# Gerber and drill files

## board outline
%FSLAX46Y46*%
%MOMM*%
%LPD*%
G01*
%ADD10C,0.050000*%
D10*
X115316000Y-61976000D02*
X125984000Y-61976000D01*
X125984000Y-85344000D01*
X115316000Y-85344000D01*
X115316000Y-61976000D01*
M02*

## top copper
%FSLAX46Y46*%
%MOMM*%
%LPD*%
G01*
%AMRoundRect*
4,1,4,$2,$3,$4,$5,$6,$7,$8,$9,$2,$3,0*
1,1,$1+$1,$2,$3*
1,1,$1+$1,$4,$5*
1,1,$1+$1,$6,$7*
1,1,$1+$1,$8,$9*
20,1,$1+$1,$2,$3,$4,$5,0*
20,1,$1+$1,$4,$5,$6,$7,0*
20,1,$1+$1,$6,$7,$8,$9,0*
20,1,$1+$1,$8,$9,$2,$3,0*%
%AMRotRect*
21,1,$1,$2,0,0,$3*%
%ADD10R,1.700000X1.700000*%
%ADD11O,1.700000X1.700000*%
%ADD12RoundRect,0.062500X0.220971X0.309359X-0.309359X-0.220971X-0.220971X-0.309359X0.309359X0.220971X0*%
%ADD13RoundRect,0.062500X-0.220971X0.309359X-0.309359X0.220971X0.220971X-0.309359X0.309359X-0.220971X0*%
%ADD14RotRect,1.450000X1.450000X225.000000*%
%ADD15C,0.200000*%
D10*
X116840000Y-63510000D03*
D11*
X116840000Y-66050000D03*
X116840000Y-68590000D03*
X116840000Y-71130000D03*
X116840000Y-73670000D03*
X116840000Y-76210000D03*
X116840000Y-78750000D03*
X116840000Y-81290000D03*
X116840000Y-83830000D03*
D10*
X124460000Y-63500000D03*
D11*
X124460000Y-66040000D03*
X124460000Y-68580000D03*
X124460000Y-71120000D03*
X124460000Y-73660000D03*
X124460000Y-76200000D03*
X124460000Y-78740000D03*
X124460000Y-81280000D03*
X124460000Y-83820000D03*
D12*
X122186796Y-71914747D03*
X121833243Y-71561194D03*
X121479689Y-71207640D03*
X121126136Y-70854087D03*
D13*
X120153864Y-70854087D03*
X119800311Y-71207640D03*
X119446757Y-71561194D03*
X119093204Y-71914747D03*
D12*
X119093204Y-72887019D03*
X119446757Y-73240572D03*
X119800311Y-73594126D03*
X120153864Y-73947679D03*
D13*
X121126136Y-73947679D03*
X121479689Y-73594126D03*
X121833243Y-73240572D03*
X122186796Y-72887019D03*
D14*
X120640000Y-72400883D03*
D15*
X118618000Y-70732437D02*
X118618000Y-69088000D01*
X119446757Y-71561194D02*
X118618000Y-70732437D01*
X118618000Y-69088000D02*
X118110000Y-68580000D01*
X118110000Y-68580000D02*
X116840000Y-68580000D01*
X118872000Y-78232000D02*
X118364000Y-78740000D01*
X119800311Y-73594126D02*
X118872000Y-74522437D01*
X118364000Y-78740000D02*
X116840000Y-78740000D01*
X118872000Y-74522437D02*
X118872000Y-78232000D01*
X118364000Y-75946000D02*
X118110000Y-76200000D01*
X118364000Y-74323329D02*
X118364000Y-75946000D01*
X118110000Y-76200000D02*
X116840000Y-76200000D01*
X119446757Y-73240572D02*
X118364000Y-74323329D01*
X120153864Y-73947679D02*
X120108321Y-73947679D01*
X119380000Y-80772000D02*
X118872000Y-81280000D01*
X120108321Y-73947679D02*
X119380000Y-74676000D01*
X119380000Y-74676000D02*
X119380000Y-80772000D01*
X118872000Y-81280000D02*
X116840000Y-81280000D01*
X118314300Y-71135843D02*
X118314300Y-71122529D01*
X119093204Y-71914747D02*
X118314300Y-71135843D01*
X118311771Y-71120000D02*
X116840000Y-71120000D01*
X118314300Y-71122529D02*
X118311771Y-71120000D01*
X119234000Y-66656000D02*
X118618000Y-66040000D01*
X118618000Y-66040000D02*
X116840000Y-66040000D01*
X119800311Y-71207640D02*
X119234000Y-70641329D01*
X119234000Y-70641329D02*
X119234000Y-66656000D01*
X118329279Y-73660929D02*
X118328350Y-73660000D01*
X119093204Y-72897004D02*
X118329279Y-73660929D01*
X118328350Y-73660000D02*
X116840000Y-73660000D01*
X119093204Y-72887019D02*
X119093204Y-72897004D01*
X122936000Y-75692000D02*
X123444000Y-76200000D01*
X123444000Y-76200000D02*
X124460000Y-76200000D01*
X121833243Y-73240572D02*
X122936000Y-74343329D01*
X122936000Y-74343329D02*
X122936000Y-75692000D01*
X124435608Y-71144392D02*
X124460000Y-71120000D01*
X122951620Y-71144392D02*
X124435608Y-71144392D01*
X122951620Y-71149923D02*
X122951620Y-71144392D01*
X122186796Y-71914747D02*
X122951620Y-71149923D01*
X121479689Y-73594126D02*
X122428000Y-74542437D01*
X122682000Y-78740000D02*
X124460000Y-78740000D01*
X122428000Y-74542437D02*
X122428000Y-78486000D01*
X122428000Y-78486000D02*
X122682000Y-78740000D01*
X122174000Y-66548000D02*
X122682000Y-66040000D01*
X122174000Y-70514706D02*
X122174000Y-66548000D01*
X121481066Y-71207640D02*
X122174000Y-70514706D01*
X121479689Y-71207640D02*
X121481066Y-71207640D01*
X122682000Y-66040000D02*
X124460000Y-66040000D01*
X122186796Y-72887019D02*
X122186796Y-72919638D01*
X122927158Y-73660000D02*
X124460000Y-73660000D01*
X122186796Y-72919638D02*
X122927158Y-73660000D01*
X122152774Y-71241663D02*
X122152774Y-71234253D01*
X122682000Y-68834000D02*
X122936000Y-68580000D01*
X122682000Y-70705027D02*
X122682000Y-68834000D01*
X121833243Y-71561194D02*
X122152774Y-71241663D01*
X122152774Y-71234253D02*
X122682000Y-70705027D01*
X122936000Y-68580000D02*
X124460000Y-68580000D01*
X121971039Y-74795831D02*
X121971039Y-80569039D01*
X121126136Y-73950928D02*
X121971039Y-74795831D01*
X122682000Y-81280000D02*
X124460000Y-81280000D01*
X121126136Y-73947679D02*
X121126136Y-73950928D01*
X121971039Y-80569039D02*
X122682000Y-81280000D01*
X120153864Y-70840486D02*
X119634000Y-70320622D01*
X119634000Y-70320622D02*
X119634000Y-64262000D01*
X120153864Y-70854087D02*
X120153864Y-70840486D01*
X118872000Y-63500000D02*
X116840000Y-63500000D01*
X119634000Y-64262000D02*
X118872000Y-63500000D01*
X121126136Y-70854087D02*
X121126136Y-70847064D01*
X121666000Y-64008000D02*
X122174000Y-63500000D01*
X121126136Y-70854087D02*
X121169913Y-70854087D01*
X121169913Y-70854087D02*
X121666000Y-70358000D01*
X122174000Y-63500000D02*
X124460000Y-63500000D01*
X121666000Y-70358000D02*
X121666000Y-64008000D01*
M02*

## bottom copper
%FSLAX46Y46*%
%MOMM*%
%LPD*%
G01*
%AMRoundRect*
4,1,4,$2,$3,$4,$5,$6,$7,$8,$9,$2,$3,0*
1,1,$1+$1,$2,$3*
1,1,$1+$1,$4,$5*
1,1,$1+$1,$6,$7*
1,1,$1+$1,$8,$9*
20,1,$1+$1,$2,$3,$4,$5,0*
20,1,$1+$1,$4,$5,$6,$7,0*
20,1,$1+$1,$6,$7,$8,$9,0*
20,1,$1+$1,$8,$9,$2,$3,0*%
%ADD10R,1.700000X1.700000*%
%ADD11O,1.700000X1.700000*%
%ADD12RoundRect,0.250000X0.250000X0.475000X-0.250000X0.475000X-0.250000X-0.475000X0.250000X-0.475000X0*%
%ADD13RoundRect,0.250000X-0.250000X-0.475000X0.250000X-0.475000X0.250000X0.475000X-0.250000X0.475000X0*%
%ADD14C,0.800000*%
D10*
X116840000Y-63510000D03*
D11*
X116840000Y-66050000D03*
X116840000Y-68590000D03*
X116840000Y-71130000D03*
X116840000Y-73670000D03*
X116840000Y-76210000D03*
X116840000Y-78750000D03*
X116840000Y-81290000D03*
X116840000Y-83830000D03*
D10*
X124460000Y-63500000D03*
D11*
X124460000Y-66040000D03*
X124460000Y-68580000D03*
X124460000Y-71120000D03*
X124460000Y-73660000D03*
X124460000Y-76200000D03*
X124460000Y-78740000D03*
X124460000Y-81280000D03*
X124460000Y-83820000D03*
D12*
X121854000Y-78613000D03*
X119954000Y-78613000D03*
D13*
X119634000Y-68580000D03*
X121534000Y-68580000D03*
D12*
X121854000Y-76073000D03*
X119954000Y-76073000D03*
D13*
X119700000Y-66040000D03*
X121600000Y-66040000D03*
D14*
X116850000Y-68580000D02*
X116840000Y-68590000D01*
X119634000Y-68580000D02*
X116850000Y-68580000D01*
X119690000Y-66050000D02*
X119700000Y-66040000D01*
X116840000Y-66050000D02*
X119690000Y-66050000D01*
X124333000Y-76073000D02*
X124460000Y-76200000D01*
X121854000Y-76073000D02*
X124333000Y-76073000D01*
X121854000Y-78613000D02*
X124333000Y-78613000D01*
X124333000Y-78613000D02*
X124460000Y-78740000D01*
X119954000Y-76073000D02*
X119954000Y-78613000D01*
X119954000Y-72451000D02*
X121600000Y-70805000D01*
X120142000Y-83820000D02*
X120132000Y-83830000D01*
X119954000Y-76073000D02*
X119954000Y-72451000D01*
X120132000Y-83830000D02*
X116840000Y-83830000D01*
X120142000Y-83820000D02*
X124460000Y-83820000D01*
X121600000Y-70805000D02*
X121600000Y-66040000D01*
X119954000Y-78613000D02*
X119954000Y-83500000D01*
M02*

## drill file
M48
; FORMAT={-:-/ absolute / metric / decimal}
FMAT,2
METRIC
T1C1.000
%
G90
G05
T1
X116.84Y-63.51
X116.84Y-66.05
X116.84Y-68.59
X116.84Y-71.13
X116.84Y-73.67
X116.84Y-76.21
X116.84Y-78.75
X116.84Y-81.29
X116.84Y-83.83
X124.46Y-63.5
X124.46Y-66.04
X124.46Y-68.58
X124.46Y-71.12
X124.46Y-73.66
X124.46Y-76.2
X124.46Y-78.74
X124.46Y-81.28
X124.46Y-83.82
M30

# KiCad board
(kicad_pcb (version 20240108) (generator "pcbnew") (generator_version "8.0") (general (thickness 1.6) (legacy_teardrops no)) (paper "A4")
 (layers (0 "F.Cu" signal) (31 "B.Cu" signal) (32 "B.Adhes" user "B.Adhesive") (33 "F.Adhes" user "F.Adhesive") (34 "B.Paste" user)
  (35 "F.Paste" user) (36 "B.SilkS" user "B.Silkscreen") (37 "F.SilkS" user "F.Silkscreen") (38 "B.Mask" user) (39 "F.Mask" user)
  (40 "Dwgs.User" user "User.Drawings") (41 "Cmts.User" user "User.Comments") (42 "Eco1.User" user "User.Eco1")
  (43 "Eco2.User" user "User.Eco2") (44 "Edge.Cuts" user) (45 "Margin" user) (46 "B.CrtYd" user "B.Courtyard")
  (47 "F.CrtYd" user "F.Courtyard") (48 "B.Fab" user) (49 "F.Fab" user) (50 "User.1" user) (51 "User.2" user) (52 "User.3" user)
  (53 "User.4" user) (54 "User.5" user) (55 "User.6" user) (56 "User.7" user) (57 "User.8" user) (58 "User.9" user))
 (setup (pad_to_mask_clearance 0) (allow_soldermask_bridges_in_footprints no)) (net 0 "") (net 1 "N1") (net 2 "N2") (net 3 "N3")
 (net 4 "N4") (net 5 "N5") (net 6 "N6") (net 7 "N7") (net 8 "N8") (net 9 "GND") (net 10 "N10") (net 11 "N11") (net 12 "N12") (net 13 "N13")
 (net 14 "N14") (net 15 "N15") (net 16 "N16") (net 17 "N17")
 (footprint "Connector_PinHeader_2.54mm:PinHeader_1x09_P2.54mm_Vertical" (layer "F.Cu") (at 116.84 63.51)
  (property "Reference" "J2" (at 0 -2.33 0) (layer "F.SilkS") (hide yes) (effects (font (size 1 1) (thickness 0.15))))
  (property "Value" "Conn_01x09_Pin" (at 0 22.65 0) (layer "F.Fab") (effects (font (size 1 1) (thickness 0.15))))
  (pad "1" thru_hole rect (at 0 0) (size 1.7 1.7) (drill 1) (layers "*.Cu" "*.Mask") (remove_unused_layers no) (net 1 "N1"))
  (pad "2" thru_hole oval (at 0 2.54) (size 1.7 1.7) (drill 1) (layers "*.Cu" "*.Mask") (remove_unused_layers no) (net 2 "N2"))
  (pad "3" thru_hole oval (at 0 5.08) (size 1.7 1.7) (drill 1) (layers "*.Cu" "*.Mask") (remove_unused_layers no) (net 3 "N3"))
  (pad "4" thru_hole oval (at 0 7.62) (size 1.7 1.7) (drill 1) (layers "*.Cu" "*.Mask") (remove_unused_layers no) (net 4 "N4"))
  (pad "5" thru_hole oval (at 0 10.16) (size 1.7 1.7) (drill 1) (layers "*.Cu" "*.Mask") (remove_unused_layers no) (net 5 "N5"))
  (pad "6" thru_hole oval (at 0 12.7) (size 1.7 1.7) (drill 1) (layers "*.Cu" "*.Mask") (remove_unused_layers no) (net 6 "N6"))
  (pad "7" thru_hole oval (at 0 15.24) (size 1.7 1.7) (drill 1) (layers "*.Cu" "*.Mask") (remove_unused_layers no) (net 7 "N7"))
  (pad "8" thru_hole oval (at 0 17.78) (size 1.7 1.7) (drill 1) (layers "*.Cu" "*.Mask") (remove_unused_layers no) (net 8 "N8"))
  (pad "9" thru_hole oval (at 0 20.32) (size 1.7 1.7) (drill 1) (layers "*.Cu" "*.Mask") (remove_unused_layers no) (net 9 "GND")))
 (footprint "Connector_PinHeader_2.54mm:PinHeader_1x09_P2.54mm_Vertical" (layer "F.Cu") (at 124.46 63.5)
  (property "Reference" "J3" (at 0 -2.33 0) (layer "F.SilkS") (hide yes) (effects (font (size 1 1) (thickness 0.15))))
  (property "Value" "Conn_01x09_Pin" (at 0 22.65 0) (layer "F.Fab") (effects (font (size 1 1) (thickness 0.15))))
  (pad "1" thru_hole rect (at 0 0) (size 1.7 1.7) (drill 1) (layers "*.Cu" "*.Mask") (remove_unused_layers no) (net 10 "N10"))
  (pad "2" thru_hole oval (at 0 2.54) (size 1.7 1.7) (drill 1) (layers "*.Cu" "*.Mask") (remove_unused_layers no) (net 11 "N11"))
  (pad "3" thru_hole oval (at 0 5.08) (size 1.7 1.7) (drill 1) (layers "*.Cu" "*.Mask") (remove_unused_layers no) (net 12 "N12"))
  (pad "4" thru_hole oval (at 0 7.62) (size 1.7 1.7) (drill 1) (layers "*.Cu" "*.Mask") (remove_unused_layers no) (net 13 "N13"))
  (pad "5" thru_hole oval (at 0 10.16) (size 1.7 1.7) (drill 1) (layers "*.Cu" "*.Mask") (remove_unused_layers no) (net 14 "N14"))
  (pad "6" thru_hole oval (at 0 12.7) (size 1.7 1.7) (drill 1) (layers "*.Cu" "*.Mask") (remove_unused_layers no) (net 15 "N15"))
  (pad "7" thru_hole oval (at 0 15.24) (size 1.7 1.7) (drill 1) (layers "*.Cu" "*.Mask") (remove_unused_layers no) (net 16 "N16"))
  (pad "8" thru_hole oval (at 0 17.78) (size 1.7 1.7) (drill 1) (layers "*.Cu" "*.Mask") (remove_unused_layers no) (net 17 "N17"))
  (pad "9" thru_hole oval (at 0 20.32) (size 1.7 1.7) (drill 1) (layers "*.Cu" "*.Mask") (remove_unused_layers no) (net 9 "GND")))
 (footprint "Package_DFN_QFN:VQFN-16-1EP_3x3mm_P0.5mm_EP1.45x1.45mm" (layer "F.Cu") (at 120.64 72.400883 -135)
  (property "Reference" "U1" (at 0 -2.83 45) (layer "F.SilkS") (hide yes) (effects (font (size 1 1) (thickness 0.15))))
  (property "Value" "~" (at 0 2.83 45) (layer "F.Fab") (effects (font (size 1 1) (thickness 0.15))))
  (pad "" smd roundrect (at -0.36 -0.36 225) (size 0.58 0.58) (layers "F.Paste") (roundrect_rratio 0.25))
  (pad "" smd roundrect (at -0.36 0.36 225) (size 0.58 0.58) (layers "F.Paste") (roundrect_rratio 0.25))
  (pad "" smd roundrect (at 0.36 -0.36 225) (size 0.58 0.58) (layers "F.Paste") (roundrect_rratio 0.25))
  (pad "" smd roundrect (at 0.36 0.36 225) (size 0.58 0.58) (layers "F.Paste") (roundrect_rratio 0.25))
  (pad "1" smd roundrect (at -1.4375 -0.75 225) (size 0.875 0.25) (layers "F.Cu" "F.Paste" "F.Mask") (roundrect_rratio 0.25) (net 13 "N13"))
  (pad "2" smd roundrect (at -1.4375 -0.25 225) (size 0.875 0.25) (layers "F.Cu" "F.Paste" "F.Mask") (roundrect_rratio 0.25) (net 12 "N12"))
  (pad "3" smd roundrect (at -1.4375 0.25 225) (size 0.875 0.25) (layers "F.Cu" "F.Paste" "F.Mask") (roundrect_rratio 0.25) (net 11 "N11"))
  (pad "4" smd roundrect (at -1.4375 0.75 225) (size 0.875 0.25) (layers "F.Cu" "F.Paste" "F.Mask") (roundrect_rratio 0.25) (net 10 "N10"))
  (pad "5" smd roundrect (at -0.75 1.4375 225) (size 0.25 0.875) (layers "F.Cu" "F.Paste" "F.Mask") (roundrect_rratio 0.25) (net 1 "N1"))
  (pad "6" smd roundrect (at -0.25 1.4375 225) (size 0.25 0.875) (layers "F.Cu" "F.Paste" "F.Mask") (roundrect_rratio 0.25) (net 2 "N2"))
  (pad "7" smd roundrect (at 0.25 1.4375 225) (size 0.25 0.875) (layers "F.Cu" "F.Paste" "F.Mask") (roundrect_rratio 0.25) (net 3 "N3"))
  (pad "8" smd roundrect (at 0.75 1.4375 225) (size 0.25 0.875) (layers "F.Cu" "F.Paste" "F.Mask") (roundrect_rratio 0.25) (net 4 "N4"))
  (pad "9" smd roundrect (at 1.4375 0.75 225) (size 0.875 0.25) (layers "F.Cu" "F.Paste" "F.Mask") (roundrect_rratio 0.25) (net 5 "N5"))
  (pad "10" smd roundrect (at 1.4375 0.25 225) (size 0.875 0.25) (layers "F.Cu" "F.Paste" "F.Mask") (roundrect_rratio 0.25) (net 6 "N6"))
  (pad "11" smd roundrect (at 1.4375 -0.25 225) (size 0.875 0.25) (layers "F.Cu" "F.Paste" "F.Mask") (roundrect_rratio 0.25) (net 7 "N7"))
  (pad "12" smd roundrect (at 1.4375 -0.75 225) (size 0.875 0.25) (layers "F.Cu" "F.Paste" "F.Mask") (roundrect_rratio 0.25) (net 8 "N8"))
  (pad "13" smd roundrect (at 0.75 -1.4375 225) (size 0.25 0.875) (layers "F.Cu" "F.Paste" "F.Mask") (roundrect_rratio 0.25) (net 17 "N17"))
  (pad "14" smd roundrect (at 0.25 -1.4375 225) (size 0.25 0.875) (layers "F.Cu" "F.Paste" "F.Mask") (roundrect_rratio 0.25) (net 16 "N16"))
  (pad "15" smd roundrect (at -0.25 -1.4375 225) (size 0.25 0.875) (layers "F.Cu" "F.Paste" "F.Mask") (roundrect_rratio 0.25) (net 15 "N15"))
  (pad "16" smd roundrect (at -0.75 -1.4375 225) (size 0.25 0.875) (layers "F.Cu" "F.Paste" "F.Mask") (roundrect_rratio 0.25) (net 14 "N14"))
  (pad "17" smd rect (at 0 0 225) (size 1.45 1.45) (layers "F.Cu" "F.Mask") (zone_connect 2)))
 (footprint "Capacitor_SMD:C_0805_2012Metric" (layer "B.Cu") (at 120.904 78.613 180)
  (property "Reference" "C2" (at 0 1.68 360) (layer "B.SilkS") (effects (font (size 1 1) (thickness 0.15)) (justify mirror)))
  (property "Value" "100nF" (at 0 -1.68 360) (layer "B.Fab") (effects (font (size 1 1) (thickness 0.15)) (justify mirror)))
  (pad "1" smd roundrect (at -0.95 0 180) (size 1 1.45) (layers "B.Cu" "B.Paste" "B.Mask") (roundrect_rratio 0.25) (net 16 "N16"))
  (pad "2" smd roundrect (at 0.95 0 180) (size 1 1.45) (layers "B.Cu" "B.Paste" "B.Mask") (roundrect_rratio 0.25) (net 9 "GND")))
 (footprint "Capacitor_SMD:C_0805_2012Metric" (layer "B.Cu") (at 120.584 68.58)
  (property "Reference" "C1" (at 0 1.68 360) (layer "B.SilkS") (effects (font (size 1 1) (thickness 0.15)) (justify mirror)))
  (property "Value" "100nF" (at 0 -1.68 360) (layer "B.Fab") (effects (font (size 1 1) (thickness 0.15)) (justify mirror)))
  (pad "1" smd roundrect (at -0.95 0) (size 1 1.45) (layers "B.Cu" "B.Paste" "B.Mask") (roundrect_rratio 0.25) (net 3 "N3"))
  (pad "2" smd roundrect (at 0.95 0) (size 1 1.45) (layers "B.Cu" "B.Paste" "B.Mask") (roundrect_rratio 0.25) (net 9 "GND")))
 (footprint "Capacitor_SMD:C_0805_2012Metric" (layer "B.Cu") (at 120.904 76.073 180)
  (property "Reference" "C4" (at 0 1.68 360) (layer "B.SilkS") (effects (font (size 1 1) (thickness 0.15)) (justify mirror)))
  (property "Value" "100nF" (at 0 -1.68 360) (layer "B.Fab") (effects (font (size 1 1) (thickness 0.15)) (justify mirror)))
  (pad "1" smd roundrect (at -0.95 0 180) (size 1 1.45) (layers "B.Cu" "B.Paste" "B.Mask") (roundrect_rratio 0.25) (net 15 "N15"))
  (pad "2" smd roundrect (at 0.95 0 180) (size 1 1.45) (layers "B.Cu" "B.Paste" "B.Mask") (roundrect_rratio 0.25) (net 9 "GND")))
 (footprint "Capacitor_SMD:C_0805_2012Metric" (layer "B.Cu") (at 120.65 66.04)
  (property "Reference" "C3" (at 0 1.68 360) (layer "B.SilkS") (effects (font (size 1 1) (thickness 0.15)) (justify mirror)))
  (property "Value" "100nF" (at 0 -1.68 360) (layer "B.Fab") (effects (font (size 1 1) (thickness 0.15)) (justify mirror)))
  (pad "1" smd roundrect (at -0.95 0) (size 1 1.45) (layers "B.Cu" "B.Paste" "B.Mask") (roundrect_rratio 0.25) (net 2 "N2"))
  (pad "2" smd roundrect (at 0.95 0) (size 1 1.45) (layers "B.Cu" "B.Paste" "B.Mask") (roundrect_rratio 0.25) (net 9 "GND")))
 (gr_rect (start 115.316 61.976) (end 125.984 85.344) (stroke (width 0.05) (type default)) (fill none) (layer "Edge.Cuts"))
 (segment (start 118.618 70.732437) (end 118.618 69.088) (width 0.2) (layer "F.Cu") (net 3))
 (segment (start 119.446757 71.561194) (end 118.618 70.732437) (width 0.2) (layer "F.Cu") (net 3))
 (segment (start 118.618 69.088) (end 118.11 68.58) (width 0.2) (layer "F.Cu") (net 3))
 (segment (start 118.11 68.58) (end 116.84 68.58) (width 0.2) (layer "F.Cu") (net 3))
 (segment (start 116.85 68.58) (end 116.84 68.59) (width 0.8) (layer "B.Cu") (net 3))
 (segment (start 119.634 68.58) (end 116.85 68.58) (width 0.8) (layer "B.Cu") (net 3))
 (segment (start 118.872 78.232) (end 118.364 78.74) (width 0.2) (layer "F.Cu") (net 7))
 (segment (start 119.800311 73.594126) (end 118.872 74.522437) (width 0.2) (layer "F.Cu") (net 7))
 (segment (start 118.364 78.74) (end 116.84 78.74) (width 0.2) (layer "F.Cu") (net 7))
 (segment (start 118.872 74.522437) (end 118.872 78.232) (width 0.2) (layer "F.Cu") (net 7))
 (segment (start 118.364 75.946) (end 118.11 76.2) (width 0.2) (layer "F.Cu") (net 6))
 (segment (start 118.364 74.323329) (end 118.364 75.946) (width 0.2) (layer "F.Cu") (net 6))
 (segment (start 118.11 76.2) (end 116.84 76.2) (width 0.2) (layer "F.Cu") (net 6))
 (segment (start 119.446757 73.240572) (end 118.364 74.323329) (width 0.2) (layer "F.Cu") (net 6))
 (segment (start 120.153864 73.947679) (end 120.108321 73.947679) (width 0.2) (layer "F.Cu") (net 8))
 (segment (start 119.38 80.772) (end 118.872 81.28) (width 0.2) (layer "F.Cu") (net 8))
 (segment (start 120.108321 73.947679) (end 119.38 74.676) (width 0.2) (layer "F.Cu") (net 8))
 (segment (start 119.38 74.676) (end 119.38 80.772) (width 0.2) (layer "F.Cu") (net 8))
 (segment (start 118.872 81.28) (end 116.84 81.28) (width 0.2) (layer "F.Cu") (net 8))
 (segment (start 118.3143 71.135843) (end 118.3143 71.122529) (width 0.2) (layer "F.Cu") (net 4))
 (segment (start 119.093204 71.914747) (end 118.3143 71.135843) (width 0.2) (layer "F.Cu") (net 4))
 (segment (start 118.311771 71.12) (end 116.84 71.12) (width 0.2) (layer "F.Cu") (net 4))
 (segment (start 118.3143 71.122529) (end 118.311771 71.12) (width 0.2) (layer "F.Cu") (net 4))
 (segment (start 119.234 66.656) (end 118.618 66.04) (width 0.2) (layer "F.Cu") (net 2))
 (segment (start 118.618 66.04) (end 116.84 66.04) (width 0.2) (layer "F.Cu") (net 2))
 (segment (start 119.800311 71.20764) (end 119.234 70.641329) (width 0.2) (layer "F.Cu") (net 2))
 (segment (start 119.234 70.641329) (end 119.234 66.656) (width 0.2) (layer "F.Cu") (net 2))
 (segment (start 119.69 66.05) (end 119.7 66.04) (width 0.8) (layer "B.Cu") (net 2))
 (segment (start 116.84 66.05) (end 119.69 66.05) (width 0.8) (layer "B.Cu") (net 2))
 (segment (start 118.329279 73.660929) (end 118.32835 73.66) (width 0.2) (layer "F.Cu") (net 5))
 (segment (start 119.093204 72.897004) (end 118.329279 73.660929) (width 0.2) (layer "F.Cu") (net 5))
 (segment (start 118.32835 73.66) (end 116.84 73.66) (width 0.2) (layer "F.Cu") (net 5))
 (segment (start 119.093204 72.887019) (end 119.093204 72.897004) (width 0.2) (layer "F.Cu") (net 5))
 (segment (start 122.936 75.692) (end 123.444 76.2) (width 0.2) (layer "F.Cu") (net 15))
 (segment (start 123.444 76.2) (end 124.46 76.2) (width 0.2) (layer "F.Cu") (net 15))
 (segment (start 121.833243 73.240572) (end 122.936 74.343329) (width 0.2) (layer "F.Cu") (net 15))
 (segment (start 122.936 74.343329) (end 122.936 75.692) (width 0.2) (layer "F.Cu") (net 15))
 (segment (start 124.333 76.073) (end 124.46 76.2) (width 0.8) (layer "B.Cu") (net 15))
 (segment (start 121.854 76.073) (end 124.333 76.073) (width 0.8) (layer "B.Cu") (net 15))
 (segment (start 124.435608 71.144392) (end 124.46 71.12) (width 0.2) (layer "F.Cu") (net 13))
 (segment (start 122.95162 71.144392) (end 124.435608 71.144392) (width 0.2) (layer "F.Cu") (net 13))
 (segment (start 122.95162 71.149923) (end 122.95162 71.144392) (width 0.2) (layer "F.Cu") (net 13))
 (segment (start 122.186796 71.914747) (end 122.95162 71.149923) (width 0.2) (layer "F.Cu") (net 13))
 (segment (start 121.479689 73.594126) (end 122.428 74.542437) (width 0.2) (layer "F.Cu") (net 16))
 (segment (start 122.682 78.74) (end 124.46 78.74) (width 0.2) (layer "F.Cu") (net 16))
 (segment (start 122.428 74.542437) (end 122.428 78.486) (width 0.2) (layer "F.Cu") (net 16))
 (segment (start 122.428 78.486) (end 122.682 78.74) (width 0.2) (layer "F.Cu") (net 16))
 (segment (start 121.854 78.613) (end 124.333 78.613) (width 0.8) (layer "B.Cu") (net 16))
 (segment (start 124.333 78.613) (end 124.46 78.74) (width 0.8) (layer "B.Cu") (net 16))
 (segment (start 122.174 66.548) (end 122.682 66.04) (width 0.2) (layer "F.Cu") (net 11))
 (segment (start 122.174 70.514706) (end 122.174 66.548) (width 0.2) (layer "F.Cu") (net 11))
 (segment (start 121.481066 71.20764) (end 122.174 70.514706) (width 0.2) (layer "F.Cu") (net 11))
 (segment (start 121.479689 71.20764) (end 121.481066 71.20764) (width 0.2) (layer "F.Cu") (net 11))
 (segment (start 122.682 66.04) (end 124.46 66.04) (width 0.2) (layer "F.Cu") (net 11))
 (segment (start 122.186796 72.887019) (end 122.186796 72.919638) (width 0.2) (layer "F.Cu") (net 14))
 (segment (start 122.927158 73.66) (end 124.46 73.66) (width 0.2) (layer "F.Cu") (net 14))
 (segment (start 122.186796 72.919638) (end 122.927158 73.66) (width 0.2) (layer "F.Cu") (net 14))
 (segment (start 122.152774 71.241663) (end 122.152774 71.234253) (width 0.2) (layer "F.Cu") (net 12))
 (segment (start 122.682 68.834) (end 122.936 68.58) (width 0.2) (layer "F.Cu") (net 12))
 (segment (start 122.682 70.705027) (end 122.682 68.834) (width 0.2) (layer "F.Cu") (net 12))
 (segment (start 121.833243 71.561194) (end 122.152774 71.241663) (width 0.2) (layer "F.Cu") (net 12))
 (segment (start 122.152774 71.234253) (end 122.682 70.705027) (width 0.2) (layer "F.Cu") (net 12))
 (segment (start 122.936 68.58) (end 124.46 68.58) (width 0.2) (layer "F.Cu") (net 12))
 (segment (start 121.971039 74.795831) (end 121.971039 80.569039) (width 0.2) (layer "F.Cu") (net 17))
 (segment (start 121.126136 73.950928) (end 121.971039 74.795831) (width 0.2) (layer "F.Cu") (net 17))
 (segment (start 122.682 81.28) (end 124.46 81.28) (width 0.2) (layer "F.Cu") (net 17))
 (segment (start 121.126136 73.947679) (end 121.126136 73.950928) (width 0.2) (layer "F.Cu") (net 17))
 (segment (start 121.971039 80.569039) (end 122.682 81.28) (width 0.2) (layer "F.Cu") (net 17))
 (segment (start 119.954 76.073) (end 119.954 78.613) (width 0.8) (layer "B.Cu") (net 9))
 (segment (start 119.954 72.451) (end 121.6 70.805) (width 0.8) (layer "B.Cu") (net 9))
 (segment (start 120.142 83.82) (end 120.132 83.83) (width 0.8) (layer "B.Cu") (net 9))
 (segment (start 119.954 76.073) (end 119.954 72.451) (width 0.8) (layer "B.Cu") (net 9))
 (segment (start 120.132 83.83) (end 116.84 83.83) (width 0.8) (layer "B.Cu") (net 9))
 (segment (start 120.142 83.82) (end 124.46 83.82) (width 0.8) (layer "B.Cu") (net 9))
 (segment (start 121.6 70.805) (end 121.6 66.04) (width 0.8) (layer "B.Cu") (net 9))
 (segment (start 119.954 78.613) (end 119.954 83.5) (width 0.8) (layer "B.Cu") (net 9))
 (segment (start 120.153864 70.840486) (end 119.634 70.320622) (width 0.2) (layer "F.Cu") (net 1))
 (segment (start 119.634 70.320622) (end 119.634 64.262) (width 0.2) (layer "F.Cu") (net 1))
 (segment (start 120.153864 70.854087) (end 120.153864 70.840486) (width 0.2) (layer "F.Cu") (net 1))
 (segment (start 118.872 63.5) (end 116.84 63.5) (width 0.2) (layer "F.Cu") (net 1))
 (segment (start 119.634 64.262) (end 118.872 63.5) (width 0.2) (layer "F.Cu") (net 1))
 (segment (start 121.126136 70.854087) (end 121.126136 70.847064) (width 0.2) (layer "F.Cu") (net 10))
 (segment (start 121.666 64.008) (end 122.174 63.5) (width 0.2) (layer "F.Cu") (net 10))
 (segment (start 121.126136 70.854087) (end 121.169913 70.854087) (width 0.2) (layer "F.Cu") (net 10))
 (segment (start 121.169913 70.854087) (end 121.666 70.358) (width 0.2) (layer "F.Cu") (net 10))
 (segment (start 122.174 63.5) (end 124.46 63.5) (width 0.2) (layer "F.Cu") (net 10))
 (segment (start 121.666 70.358) (end 121.666 64.008) (width 0.2) (layer "F.Cu") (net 10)))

